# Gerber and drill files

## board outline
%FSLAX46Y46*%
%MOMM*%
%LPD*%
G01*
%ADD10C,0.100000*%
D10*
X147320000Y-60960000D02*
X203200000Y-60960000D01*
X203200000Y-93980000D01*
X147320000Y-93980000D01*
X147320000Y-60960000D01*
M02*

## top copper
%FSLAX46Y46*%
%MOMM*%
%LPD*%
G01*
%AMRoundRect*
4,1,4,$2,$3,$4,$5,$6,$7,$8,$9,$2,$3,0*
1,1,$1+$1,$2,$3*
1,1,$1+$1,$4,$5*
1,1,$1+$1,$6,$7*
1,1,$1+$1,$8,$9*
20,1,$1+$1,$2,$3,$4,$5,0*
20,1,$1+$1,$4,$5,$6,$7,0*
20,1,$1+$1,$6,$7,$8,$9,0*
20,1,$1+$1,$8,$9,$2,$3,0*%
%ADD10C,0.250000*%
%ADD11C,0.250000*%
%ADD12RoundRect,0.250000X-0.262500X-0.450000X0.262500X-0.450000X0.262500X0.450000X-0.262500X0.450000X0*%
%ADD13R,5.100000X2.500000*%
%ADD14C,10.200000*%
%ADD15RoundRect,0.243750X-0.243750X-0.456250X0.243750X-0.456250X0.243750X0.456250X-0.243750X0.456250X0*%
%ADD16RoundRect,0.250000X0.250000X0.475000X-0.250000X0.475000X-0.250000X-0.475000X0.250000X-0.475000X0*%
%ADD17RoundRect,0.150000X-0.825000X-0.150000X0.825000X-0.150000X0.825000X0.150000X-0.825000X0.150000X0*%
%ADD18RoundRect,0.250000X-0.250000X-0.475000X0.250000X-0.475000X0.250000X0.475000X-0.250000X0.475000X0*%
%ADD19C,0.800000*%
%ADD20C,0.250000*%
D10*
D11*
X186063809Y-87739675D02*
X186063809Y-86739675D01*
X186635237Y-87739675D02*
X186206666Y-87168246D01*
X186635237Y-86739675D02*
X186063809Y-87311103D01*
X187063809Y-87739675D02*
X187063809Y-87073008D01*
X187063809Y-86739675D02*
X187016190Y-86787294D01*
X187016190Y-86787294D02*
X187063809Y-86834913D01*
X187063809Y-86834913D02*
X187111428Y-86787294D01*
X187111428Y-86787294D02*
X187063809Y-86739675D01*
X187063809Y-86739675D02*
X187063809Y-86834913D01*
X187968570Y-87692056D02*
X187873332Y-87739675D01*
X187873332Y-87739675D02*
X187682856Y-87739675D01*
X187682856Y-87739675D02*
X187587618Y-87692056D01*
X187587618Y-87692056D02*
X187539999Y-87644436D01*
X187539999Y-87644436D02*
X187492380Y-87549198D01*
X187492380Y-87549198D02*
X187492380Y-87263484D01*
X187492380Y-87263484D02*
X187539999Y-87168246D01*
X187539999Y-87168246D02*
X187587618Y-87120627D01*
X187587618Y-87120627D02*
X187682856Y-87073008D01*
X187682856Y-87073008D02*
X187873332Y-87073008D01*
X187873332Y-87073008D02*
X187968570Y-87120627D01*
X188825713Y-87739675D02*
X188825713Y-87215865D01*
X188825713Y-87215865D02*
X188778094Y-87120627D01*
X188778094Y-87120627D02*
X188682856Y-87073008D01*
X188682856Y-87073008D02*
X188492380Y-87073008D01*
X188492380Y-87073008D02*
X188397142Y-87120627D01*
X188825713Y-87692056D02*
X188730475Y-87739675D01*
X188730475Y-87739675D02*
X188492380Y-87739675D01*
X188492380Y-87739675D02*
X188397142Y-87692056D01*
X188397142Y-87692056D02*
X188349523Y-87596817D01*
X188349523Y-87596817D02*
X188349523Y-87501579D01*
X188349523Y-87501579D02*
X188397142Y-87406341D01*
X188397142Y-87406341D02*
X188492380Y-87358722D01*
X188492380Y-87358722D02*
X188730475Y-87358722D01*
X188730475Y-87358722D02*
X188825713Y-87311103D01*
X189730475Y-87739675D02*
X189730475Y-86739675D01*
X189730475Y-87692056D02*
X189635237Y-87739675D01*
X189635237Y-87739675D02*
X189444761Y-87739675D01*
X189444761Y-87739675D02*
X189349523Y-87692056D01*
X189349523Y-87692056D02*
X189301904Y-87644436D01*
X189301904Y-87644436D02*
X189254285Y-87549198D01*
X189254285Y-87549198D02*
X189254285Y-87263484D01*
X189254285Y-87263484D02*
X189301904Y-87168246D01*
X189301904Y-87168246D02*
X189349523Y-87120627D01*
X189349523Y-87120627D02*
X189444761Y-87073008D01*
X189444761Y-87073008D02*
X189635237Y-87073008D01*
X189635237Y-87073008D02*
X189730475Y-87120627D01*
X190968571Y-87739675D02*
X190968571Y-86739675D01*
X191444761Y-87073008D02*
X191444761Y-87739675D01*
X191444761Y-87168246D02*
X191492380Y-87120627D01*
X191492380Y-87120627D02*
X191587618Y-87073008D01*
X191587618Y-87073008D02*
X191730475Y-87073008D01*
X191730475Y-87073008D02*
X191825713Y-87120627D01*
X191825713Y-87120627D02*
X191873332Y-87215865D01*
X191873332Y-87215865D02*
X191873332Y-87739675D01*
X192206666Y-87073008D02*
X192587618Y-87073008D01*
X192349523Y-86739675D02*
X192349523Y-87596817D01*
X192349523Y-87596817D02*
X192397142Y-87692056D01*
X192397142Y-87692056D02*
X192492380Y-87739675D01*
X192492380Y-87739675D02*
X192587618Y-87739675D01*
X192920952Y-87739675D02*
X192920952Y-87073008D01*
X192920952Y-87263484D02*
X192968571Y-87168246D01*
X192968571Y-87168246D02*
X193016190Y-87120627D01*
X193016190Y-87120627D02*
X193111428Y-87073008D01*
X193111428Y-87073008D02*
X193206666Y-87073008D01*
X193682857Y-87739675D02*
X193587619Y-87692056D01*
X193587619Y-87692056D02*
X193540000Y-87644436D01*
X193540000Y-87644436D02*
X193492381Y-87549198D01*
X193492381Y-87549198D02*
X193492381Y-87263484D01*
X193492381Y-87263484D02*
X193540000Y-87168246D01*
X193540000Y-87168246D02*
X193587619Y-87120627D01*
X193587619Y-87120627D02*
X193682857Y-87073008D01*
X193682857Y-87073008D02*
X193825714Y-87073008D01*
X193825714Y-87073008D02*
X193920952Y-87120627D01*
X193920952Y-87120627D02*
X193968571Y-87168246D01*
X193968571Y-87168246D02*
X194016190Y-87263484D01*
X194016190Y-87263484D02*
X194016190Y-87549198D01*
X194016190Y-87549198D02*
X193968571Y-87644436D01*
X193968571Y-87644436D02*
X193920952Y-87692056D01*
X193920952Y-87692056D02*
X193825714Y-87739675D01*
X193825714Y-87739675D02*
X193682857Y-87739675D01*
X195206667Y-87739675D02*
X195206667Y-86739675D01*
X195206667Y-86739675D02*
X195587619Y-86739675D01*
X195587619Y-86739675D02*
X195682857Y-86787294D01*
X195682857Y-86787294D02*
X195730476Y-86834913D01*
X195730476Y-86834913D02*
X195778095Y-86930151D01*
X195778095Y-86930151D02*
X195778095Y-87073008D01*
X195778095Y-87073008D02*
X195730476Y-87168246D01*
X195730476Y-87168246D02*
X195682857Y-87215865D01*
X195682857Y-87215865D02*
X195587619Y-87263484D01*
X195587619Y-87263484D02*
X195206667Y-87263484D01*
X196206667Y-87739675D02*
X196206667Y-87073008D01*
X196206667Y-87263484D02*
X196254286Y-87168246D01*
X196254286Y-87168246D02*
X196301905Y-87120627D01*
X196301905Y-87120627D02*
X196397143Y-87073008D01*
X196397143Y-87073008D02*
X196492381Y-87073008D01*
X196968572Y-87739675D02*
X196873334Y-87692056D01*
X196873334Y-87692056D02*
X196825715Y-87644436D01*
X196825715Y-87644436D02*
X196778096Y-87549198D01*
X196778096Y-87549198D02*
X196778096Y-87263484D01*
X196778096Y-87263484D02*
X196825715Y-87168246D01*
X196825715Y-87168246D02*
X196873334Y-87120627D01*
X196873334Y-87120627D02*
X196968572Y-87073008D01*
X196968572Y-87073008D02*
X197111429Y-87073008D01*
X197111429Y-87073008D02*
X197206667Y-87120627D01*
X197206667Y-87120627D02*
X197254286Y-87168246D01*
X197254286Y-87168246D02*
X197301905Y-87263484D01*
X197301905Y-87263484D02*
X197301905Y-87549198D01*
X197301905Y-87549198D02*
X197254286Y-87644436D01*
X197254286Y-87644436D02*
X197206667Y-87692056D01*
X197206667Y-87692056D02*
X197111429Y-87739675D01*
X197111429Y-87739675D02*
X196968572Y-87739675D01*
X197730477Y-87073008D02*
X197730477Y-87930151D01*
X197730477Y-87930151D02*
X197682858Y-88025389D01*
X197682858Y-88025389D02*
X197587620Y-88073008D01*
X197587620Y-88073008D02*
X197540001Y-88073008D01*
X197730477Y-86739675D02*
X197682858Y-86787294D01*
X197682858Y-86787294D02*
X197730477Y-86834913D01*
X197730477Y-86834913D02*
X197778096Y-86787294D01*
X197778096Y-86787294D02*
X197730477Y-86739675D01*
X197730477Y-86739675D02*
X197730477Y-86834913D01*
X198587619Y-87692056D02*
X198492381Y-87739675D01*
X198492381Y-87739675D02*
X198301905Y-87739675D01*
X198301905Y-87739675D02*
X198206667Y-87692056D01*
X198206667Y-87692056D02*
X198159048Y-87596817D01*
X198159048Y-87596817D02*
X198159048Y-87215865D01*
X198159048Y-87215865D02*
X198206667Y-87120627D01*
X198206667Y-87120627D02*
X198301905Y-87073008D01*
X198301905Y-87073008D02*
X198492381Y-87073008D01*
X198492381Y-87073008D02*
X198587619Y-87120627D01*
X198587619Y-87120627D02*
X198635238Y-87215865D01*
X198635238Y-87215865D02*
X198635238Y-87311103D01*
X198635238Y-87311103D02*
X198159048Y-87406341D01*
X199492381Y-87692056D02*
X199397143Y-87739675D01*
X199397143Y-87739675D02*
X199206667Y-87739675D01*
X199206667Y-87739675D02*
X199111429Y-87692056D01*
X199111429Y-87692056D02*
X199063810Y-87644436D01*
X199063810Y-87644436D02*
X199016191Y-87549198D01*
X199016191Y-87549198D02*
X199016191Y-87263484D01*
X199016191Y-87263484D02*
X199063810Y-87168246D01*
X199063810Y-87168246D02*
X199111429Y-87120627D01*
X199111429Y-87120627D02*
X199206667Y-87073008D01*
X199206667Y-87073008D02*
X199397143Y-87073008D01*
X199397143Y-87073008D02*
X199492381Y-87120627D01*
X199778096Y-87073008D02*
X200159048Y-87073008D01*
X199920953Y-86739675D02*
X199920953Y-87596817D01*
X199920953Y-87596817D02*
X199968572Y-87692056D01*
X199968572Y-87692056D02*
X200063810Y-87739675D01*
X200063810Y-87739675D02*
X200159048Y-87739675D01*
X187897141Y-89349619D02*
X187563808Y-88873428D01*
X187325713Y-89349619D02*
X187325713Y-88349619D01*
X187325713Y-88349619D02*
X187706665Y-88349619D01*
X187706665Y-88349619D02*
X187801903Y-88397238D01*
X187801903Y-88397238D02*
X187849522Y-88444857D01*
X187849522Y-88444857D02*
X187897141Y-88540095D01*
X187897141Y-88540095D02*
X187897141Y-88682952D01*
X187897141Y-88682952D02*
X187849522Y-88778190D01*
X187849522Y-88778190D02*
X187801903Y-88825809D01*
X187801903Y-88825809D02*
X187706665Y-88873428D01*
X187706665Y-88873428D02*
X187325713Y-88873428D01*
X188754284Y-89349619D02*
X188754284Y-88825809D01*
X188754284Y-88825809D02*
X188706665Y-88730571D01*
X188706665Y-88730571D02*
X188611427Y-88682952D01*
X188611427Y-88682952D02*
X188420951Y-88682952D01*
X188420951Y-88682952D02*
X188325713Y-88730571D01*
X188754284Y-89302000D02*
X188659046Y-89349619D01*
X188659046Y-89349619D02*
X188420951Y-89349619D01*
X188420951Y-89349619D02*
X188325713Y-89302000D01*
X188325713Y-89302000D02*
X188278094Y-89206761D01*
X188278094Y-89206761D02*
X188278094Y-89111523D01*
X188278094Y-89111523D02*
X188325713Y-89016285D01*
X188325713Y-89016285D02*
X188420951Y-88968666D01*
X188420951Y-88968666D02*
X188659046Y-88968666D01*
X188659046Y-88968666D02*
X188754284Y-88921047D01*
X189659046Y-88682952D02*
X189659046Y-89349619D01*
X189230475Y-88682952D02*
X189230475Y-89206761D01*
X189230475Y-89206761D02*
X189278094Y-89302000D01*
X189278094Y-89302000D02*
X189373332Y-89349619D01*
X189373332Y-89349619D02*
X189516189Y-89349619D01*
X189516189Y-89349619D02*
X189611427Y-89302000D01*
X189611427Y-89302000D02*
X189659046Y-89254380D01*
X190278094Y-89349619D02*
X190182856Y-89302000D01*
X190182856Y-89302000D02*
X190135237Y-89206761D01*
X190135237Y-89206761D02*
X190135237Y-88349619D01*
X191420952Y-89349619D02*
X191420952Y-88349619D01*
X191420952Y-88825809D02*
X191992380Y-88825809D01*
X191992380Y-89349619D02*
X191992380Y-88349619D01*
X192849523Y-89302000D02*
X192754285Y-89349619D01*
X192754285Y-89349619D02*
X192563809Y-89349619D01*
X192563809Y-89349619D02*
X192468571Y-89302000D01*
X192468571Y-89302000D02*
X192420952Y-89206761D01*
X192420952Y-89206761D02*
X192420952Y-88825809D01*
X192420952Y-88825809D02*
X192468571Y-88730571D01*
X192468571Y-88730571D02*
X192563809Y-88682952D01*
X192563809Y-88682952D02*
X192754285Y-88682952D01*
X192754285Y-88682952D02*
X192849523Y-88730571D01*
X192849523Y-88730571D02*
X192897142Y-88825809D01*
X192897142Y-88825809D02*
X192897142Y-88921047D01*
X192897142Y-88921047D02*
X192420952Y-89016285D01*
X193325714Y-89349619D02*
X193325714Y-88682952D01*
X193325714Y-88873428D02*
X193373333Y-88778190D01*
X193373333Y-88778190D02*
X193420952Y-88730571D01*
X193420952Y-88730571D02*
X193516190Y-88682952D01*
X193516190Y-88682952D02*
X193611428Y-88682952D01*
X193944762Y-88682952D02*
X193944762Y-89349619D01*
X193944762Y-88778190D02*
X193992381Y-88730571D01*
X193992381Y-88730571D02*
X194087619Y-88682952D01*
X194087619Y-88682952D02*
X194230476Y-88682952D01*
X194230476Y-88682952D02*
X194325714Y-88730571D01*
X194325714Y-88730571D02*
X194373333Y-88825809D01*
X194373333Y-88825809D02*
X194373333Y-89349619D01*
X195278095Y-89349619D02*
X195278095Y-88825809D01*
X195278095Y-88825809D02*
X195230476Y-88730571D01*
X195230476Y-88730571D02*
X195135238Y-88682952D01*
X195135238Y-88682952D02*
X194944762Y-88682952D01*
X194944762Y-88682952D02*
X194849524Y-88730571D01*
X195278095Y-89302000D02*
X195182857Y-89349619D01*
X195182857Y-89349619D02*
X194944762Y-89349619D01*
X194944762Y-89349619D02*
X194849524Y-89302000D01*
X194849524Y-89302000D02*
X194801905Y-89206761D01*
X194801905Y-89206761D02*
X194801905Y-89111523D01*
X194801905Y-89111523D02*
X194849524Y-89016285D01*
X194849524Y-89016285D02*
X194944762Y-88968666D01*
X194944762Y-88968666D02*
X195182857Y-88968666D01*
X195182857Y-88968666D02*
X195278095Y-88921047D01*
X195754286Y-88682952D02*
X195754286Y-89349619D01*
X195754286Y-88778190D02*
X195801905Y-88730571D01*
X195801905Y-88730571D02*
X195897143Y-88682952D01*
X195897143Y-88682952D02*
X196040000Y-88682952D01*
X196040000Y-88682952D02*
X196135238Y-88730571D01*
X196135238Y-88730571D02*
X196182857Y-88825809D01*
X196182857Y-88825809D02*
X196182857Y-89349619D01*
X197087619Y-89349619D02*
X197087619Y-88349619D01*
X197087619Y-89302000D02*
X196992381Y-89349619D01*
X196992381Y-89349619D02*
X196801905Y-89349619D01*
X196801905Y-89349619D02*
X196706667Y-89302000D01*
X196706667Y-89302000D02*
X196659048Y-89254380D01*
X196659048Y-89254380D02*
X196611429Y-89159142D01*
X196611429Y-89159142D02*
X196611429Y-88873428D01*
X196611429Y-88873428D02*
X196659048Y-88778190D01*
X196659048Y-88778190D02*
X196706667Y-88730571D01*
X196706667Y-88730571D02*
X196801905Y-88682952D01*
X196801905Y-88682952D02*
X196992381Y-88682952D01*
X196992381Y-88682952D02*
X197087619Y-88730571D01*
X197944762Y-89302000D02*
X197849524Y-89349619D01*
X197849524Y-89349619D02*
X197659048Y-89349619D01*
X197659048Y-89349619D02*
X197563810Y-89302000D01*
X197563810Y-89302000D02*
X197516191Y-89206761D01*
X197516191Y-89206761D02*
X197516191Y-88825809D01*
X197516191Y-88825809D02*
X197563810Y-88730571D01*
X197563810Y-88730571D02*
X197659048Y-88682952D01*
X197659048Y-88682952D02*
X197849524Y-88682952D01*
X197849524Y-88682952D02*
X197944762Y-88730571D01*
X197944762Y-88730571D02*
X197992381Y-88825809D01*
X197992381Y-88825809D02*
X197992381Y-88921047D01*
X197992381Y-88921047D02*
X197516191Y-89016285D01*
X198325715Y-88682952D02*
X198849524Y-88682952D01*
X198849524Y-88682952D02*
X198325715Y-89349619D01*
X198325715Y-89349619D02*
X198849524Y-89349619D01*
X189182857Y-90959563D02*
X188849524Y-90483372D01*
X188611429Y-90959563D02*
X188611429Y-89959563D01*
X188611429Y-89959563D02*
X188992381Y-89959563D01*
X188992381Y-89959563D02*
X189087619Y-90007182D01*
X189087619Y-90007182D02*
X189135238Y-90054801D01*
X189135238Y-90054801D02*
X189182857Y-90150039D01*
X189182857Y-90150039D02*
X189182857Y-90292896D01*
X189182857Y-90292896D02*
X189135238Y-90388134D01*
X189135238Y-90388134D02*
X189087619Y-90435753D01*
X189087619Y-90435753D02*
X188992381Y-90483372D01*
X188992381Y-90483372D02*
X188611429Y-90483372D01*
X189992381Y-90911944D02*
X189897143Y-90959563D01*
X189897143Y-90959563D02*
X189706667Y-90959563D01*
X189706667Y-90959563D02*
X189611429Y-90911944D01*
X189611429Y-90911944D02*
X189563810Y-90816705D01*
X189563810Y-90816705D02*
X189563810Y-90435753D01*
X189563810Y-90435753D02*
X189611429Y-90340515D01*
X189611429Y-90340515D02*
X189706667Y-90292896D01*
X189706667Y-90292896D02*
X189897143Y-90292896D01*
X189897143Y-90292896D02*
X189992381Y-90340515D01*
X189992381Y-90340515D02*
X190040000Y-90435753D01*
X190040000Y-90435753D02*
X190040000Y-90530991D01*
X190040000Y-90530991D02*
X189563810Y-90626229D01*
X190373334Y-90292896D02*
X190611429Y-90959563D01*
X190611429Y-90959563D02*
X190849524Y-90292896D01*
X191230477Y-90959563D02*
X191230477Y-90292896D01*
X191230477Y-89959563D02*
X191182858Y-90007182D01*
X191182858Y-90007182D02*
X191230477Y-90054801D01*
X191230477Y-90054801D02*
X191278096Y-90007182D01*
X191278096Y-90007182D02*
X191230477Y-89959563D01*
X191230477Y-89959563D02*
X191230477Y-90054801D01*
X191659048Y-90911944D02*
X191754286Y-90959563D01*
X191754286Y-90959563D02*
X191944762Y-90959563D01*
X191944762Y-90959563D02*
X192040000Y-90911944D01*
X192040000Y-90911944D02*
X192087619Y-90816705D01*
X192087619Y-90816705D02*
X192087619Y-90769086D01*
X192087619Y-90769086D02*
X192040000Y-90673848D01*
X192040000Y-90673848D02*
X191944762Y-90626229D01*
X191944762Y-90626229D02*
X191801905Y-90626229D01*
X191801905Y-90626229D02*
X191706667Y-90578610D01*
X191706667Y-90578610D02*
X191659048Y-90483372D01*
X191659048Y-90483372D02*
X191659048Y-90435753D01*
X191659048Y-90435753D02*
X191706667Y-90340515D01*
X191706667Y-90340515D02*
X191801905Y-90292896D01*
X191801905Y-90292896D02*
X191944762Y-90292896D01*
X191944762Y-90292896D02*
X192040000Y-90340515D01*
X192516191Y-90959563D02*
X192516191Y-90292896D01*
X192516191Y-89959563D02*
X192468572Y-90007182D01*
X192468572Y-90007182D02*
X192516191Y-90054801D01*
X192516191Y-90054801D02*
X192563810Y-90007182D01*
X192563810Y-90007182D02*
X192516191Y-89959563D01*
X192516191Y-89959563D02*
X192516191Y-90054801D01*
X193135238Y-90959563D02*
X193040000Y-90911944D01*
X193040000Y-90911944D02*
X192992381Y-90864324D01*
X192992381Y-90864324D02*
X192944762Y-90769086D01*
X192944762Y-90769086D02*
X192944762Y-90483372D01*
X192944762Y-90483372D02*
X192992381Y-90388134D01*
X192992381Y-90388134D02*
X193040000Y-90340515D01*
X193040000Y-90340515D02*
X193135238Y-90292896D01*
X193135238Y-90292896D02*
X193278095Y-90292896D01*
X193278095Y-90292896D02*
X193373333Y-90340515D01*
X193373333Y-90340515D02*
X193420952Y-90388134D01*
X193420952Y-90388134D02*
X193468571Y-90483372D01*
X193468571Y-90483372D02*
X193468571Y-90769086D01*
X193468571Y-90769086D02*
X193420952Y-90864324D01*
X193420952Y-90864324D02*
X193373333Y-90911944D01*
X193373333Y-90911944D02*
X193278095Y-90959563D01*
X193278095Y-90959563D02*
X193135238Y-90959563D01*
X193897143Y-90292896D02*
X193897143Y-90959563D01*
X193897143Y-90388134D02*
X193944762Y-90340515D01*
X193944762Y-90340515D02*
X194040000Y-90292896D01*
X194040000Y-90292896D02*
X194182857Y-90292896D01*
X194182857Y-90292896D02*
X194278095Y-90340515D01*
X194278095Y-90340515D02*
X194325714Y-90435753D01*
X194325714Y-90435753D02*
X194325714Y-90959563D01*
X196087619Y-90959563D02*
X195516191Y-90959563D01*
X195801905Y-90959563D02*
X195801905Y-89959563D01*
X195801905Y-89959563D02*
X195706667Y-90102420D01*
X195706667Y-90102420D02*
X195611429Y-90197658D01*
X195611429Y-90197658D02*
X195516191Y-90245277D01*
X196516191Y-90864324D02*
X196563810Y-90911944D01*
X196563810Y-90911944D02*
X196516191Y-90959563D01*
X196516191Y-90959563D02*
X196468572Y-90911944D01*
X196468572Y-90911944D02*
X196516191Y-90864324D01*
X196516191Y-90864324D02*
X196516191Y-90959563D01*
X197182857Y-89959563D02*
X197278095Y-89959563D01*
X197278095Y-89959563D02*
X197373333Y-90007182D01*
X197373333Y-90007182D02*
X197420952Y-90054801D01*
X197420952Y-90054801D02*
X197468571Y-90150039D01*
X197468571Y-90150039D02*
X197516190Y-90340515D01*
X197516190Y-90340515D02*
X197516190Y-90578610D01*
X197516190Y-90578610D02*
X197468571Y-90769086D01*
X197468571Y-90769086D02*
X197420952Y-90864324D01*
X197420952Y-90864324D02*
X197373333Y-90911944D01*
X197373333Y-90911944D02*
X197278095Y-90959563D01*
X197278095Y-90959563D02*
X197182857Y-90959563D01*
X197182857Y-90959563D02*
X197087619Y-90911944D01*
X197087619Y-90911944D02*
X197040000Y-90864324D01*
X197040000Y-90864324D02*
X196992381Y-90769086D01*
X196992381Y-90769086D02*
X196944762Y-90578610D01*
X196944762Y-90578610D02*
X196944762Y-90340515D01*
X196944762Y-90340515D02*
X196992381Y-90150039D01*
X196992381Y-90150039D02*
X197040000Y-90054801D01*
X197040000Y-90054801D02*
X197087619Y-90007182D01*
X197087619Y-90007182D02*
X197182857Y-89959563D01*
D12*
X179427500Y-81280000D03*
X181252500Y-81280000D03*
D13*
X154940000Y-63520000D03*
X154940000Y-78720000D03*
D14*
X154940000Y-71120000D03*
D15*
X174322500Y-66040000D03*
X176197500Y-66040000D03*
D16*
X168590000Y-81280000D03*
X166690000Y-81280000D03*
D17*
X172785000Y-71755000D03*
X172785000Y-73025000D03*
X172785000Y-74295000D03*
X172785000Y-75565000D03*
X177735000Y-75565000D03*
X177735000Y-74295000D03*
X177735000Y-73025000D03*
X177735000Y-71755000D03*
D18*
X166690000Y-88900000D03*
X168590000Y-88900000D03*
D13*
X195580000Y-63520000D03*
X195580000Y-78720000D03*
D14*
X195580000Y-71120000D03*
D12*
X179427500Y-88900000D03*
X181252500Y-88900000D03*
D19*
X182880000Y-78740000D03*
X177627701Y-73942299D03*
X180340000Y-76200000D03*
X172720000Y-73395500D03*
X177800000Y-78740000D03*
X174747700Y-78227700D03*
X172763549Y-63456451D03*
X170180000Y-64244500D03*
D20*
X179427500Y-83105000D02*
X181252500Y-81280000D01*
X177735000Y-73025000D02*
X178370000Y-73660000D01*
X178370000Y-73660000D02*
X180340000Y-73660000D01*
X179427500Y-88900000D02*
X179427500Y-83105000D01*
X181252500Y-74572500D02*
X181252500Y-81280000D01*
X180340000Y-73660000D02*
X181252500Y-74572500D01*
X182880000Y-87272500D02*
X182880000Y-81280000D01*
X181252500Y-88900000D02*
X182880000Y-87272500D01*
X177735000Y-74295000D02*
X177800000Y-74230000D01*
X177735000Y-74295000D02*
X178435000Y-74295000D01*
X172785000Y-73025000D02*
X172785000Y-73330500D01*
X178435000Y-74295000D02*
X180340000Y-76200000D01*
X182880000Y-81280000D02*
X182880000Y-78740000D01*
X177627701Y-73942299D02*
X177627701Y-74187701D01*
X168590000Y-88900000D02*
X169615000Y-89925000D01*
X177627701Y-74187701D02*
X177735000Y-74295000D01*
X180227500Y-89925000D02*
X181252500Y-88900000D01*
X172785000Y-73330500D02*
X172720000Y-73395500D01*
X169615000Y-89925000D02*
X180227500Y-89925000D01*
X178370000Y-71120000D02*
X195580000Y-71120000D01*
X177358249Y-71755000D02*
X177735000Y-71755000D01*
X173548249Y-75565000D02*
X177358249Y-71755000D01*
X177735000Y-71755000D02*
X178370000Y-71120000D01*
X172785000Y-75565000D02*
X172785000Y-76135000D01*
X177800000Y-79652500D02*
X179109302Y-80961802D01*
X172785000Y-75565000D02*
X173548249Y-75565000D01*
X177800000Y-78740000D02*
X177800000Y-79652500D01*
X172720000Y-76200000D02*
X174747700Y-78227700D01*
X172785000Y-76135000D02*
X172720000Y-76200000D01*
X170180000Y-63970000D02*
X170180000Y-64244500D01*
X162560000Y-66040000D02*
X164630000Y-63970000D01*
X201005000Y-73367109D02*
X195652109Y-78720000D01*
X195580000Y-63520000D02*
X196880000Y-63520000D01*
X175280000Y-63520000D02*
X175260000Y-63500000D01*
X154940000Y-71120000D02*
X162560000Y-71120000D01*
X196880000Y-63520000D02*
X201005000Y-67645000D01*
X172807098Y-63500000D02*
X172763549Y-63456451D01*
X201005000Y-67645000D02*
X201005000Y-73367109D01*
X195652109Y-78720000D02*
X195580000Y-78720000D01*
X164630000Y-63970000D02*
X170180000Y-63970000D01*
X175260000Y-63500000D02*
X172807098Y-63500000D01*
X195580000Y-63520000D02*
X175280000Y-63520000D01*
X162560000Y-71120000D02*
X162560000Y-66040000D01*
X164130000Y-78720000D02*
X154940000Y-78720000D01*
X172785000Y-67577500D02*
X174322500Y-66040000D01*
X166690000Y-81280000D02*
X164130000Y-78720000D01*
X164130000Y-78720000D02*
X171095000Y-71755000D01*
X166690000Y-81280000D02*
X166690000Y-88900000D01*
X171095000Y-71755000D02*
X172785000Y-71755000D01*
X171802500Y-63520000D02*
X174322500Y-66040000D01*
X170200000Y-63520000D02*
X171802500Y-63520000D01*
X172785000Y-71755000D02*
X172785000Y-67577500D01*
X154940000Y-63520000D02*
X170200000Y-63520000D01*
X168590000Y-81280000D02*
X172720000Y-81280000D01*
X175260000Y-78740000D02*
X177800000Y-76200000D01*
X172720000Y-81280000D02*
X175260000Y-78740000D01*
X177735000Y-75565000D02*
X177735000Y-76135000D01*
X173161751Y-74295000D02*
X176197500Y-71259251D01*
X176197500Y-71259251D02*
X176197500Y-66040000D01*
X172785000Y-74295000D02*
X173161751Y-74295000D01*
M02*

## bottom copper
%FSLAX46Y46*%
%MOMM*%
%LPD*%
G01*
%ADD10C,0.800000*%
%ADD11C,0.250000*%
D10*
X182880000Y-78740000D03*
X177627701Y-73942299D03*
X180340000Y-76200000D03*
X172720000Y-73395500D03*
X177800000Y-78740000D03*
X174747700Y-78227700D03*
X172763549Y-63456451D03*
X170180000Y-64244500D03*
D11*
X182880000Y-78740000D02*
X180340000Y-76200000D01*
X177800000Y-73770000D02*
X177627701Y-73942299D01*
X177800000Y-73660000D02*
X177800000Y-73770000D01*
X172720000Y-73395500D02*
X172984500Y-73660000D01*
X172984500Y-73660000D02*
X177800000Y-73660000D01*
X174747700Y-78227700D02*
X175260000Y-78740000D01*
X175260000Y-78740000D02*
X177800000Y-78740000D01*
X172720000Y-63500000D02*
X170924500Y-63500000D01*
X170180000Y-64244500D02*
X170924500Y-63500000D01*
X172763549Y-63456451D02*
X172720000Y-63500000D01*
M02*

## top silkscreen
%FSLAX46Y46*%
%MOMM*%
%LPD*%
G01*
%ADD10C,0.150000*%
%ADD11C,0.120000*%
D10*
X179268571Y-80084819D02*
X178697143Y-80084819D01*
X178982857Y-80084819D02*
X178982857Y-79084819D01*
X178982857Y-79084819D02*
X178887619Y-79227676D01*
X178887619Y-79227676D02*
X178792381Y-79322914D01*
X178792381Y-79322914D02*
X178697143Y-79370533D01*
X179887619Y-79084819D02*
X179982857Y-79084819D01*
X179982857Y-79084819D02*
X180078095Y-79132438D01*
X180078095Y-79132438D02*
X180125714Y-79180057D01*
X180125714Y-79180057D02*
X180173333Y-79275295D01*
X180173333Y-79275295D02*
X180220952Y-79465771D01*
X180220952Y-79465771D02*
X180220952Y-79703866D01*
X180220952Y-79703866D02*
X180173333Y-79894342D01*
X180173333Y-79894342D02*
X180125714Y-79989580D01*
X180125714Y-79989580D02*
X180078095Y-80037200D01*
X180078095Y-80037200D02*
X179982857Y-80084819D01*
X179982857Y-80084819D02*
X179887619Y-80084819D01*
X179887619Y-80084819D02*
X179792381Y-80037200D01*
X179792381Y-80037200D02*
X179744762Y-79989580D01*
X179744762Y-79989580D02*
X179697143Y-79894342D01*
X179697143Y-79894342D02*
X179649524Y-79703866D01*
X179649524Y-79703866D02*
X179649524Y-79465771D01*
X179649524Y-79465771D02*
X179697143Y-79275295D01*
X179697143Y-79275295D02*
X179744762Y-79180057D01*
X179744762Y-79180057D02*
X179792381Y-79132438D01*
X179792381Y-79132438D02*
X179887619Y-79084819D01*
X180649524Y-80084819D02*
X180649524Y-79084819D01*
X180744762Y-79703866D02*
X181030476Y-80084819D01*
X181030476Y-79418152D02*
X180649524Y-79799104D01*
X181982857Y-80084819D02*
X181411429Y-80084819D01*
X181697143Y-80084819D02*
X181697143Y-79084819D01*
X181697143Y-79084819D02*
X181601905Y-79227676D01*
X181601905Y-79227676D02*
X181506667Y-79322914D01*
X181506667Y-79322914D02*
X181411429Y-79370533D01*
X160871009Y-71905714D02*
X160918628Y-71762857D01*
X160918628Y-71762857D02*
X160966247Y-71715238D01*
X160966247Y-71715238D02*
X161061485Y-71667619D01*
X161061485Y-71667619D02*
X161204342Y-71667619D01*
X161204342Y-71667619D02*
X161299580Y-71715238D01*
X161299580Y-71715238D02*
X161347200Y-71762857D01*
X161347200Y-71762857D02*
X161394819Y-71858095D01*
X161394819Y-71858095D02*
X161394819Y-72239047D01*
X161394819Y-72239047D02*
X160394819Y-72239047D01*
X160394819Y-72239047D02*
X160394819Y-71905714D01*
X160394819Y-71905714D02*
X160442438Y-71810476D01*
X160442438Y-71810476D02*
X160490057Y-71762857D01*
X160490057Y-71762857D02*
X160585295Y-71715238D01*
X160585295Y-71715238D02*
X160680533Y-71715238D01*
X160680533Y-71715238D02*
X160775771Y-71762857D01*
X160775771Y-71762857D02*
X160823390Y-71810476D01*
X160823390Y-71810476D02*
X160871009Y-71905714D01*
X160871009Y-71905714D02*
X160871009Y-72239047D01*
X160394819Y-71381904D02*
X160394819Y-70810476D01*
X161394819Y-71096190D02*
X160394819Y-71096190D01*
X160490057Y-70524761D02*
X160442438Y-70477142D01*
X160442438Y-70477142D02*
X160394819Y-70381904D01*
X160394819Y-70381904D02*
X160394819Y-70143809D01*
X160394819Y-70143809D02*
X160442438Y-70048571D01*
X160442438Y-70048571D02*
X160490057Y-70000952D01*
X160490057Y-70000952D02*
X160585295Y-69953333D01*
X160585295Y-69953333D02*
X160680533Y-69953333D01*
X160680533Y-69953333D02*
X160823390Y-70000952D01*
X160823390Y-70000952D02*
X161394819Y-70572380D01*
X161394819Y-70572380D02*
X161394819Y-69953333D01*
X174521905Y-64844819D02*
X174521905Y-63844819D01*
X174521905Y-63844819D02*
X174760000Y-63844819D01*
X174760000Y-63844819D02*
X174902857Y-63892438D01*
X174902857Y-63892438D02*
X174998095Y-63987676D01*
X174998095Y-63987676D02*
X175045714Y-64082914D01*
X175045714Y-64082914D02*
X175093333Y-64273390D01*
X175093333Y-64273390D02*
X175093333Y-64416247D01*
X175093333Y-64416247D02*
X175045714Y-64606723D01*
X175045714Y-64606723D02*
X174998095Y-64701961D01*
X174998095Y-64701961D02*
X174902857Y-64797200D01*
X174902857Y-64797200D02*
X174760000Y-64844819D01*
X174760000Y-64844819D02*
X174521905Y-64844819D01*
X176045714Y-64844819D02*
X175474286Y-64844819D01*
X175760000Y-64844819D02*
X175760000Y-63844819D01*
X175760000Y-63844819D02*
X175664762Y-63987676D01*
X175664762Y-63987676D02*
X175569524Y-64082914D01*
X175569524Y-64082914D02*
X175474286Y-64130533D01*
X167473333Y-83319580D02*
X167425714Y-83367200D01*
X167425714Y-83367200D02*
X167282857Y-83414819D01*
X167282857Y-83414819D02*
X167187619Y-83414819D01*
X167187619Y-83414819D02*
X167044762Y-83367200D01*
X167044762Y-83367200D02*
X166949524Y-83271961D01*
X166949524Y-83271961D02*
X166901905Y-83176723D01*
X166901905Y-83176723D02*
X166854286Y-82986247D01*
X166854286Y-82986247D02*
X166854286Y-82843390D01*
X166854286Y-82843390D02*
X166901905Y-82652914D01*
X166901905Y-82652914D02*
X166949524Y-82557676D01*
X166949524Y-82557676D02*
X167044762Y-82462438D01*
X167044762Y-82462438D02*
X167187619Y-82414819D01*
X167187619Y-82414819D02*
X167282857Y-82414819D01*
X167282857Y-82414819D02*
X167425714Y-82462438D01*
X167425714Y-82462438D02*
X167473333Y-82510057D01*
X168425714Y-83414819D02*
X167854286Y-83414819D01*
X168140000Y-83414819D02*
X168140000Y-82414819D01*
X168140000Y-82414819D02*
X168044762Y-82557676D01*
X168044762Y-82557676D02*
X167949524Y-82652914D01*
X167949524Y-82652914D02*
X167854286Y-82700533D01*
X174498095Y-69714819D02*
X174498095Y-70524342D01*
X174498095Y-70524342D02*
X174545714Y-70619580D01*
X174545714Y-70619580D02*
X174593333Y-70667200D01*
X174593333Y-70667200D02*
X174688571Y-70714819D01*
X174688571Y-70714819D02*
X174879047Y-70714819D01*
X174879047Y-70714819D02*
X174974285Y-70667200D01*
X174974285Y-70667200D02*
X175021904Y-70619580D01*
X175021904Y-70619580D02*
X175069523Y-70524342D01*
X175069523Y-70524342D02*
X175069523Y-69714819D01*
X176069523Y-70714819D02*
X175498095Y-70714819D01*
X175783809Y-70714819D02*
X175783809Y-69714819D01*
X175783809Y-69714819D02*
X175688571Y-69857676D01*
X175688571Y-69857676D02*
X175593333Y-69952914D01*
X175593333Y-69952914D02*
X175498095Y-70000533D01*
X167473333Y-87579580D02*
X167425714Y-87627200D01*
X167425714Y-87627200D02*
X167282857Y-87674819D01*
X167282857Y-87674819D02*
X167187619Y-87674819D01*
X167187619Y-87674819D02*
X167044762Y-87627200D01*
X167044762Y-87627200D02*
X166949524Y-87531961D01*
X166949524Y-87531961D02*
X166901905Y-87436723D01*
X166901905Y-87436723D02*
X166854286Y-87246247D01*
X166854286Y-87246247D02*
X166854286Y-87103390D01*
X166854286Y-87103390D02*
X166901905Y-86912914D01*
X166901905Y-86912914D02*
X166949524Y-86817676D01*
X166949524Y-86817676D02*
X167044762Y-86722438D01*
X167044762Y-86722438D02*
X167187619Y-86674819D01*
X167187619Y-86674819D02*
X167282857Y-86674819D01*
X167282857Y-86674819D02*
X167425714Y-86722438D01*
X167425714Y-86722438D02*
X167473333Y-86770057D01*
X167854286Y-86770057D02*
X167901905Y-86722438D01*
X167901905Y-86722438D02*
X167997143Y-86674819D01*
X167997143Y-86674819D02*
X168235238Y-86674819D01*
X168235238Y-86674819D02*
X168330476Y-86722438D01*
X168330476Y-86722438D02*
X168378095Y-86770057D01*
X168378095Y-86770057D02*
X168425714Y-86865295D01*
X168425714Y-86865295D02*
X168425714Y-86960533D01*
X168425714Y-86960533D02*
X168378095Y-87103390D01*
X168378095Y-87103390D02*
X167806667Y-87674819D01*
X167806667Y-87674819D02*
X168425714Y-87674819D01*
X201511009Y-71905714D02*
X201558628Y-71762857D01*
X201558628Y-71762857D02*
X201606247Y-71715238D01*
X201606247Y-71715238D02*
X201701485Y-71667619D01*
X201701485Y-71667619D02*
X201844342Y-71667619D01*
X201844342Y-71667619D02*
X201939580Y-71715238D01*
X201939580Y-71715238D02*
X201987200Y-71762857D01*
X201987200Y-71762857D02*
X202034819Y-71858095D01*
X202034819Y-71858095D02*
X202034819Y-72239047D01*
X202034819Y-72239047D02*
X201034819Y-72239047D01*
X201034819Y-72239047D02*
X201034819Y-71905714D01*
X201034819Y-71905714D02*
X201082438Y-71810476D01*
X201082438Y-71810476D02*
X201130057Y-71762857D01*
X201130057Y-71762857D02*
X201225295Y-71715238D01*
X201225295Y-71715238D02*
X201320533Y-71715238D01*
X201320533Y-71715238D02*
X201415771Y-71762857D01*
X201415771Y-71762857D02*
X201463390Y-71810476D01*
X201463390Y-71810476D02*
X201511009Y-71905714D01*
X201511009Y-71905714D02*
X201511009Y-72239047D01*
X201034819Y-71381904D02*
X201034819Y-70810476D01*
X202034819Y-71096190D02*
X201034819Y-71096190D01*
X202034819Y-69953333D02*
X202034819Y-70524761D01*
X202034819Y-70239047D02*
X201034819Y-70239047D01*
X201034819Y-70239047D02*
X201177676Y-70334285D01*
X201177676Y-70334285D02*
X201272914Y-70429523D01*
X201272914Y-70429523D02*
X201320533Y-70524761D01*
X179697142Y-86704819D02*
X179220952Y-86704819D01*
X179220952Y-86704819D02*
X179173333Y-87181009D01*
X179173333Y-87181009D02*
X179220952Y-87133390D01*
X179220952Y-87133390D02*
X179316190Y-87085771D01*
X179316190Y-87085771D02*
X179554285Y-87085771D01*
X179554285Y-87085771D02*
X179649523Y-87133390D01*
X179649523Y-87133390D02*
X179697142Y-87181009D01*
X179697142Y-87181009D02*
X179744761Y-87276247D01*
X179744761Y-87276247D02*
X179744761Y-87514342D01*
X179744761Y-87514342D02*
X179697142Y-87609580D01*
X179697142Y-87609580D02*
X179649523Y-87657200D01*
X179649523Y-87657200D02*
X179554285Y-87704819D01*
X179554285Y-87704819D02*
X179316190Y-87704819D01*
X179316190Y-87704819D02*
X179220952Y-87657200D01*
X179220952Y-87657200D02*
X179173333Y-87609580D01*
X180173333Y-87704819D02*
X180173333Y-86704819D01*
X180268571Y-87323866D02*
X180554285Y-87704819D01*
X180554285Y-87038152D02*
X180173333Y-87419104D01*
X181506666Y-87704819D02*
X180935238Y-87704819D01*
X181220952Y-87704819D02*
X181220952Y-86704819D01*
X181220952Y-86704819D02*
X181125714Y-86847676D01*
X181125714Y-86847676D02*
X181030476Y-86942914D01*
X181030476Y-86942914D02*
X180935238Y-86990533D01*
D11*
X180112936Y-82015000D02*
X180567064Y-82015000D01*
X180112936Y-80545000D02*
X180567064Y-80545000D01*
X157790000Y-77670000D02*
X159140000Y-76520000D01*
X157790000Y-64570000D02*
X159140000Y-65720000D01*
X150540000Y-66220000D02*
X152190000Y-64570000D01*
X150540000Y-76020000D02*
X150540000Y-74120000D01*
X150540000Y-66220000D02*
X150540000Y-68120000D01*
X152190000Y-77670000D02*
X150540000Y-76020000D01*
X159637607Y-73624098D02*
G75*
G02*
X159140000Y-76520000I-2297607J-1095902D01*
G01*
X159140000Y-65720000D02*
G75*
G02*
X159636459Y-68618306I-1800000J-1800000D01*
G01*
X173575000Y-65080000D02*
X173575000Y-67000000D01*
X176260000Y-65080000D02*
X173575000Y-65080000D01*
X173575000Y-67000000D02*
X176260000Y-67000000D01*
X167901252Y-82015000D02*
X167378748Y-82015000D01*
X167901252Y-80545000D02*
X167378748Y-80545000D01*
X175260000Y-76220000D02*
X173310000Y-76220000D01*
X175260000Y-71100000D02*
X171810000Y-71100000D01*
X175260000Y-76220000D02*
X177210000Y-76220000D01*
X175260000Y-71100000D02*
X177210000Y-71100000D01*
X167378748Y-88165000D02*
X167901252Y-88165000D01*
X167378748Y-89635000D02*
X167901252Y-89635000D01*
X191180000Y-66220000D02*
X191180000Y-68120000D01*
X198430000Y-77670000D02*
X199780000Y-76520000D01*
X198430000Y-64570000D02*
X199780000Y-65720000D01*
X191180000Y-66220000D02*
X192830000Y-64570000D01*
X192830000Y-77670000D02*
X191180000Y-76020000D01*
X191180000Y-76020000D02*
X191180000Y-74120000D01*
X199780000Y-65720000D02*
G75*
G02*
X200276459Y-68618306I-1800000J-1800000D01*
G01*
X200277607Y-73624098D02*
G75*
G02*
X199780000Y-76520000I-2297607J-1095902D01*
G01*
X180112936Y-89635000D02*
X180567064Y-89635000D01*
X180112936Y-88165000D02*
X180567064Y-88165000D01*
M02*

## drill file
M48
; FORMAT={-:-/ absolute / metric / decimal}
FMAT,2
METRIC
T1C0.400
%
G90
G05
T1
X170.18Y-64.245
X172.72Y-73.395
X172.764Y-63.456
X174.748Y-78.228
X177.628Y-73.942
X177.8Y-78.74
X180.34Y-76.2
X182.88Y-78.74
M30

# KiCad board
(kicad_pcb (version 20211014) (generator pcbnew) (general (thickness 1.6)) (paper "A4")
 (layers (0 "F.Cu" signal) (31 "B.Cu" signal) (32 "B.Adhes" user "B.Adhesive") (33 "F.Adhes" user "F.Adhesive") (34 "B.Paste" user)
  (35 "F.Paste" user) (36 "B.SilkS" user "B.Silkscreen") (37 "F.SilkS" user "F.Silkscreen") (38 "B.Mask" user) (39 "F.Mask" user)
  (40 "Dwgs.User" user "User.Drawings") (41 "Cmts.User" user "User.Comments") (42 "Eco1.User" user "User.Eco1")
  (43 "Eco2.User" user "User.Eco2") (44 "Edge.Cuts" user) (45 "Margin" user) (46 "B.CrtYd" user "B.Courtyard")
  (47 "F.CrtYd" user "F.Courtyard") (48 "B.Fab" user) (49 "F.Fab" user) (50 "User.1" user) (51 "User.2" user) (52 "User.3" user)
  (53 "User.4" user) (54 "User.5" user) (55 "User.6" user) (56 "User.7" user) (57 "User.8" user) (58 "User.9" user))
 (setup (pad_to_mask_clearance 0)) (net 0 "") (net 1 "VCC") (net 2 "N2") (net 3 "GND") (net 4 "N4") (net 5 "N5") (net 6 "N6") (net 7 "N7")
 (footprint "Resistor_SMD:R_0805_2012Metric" (layer "F.Cu") (at 180.34 81.28)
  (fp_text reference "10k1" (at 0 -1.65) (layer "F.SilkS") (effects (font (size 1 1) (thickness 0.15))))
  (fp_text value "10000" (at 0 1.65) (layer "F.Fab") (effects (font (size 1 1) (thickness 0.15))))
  (fp_line (start -0.227064 0.735) (end 0.227064 0.735) (layer "F.SilkS") (width 0.12))
  (fp_line (start -0.227064 -0.735) (end 0.227064 -0.735) (layer "F.SilkS") (width 0.12))
  (pad "1" smd roundrect (at -0.9125 0) (size 1.025 1.4) (layers "F.Cu" "F.Paste" "F.Mask") (roundrect_rratio 0.243902439) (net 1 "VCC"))
  (pad "2" smd roundrect (at 0.9125 0) (size 1.025 1.4) (layers "F.Cu" "F.Paste" "F.Mask") (roundrect_rratio 0.243902439) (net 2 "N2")))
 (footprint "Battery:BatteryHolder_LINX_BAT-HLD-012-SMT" (layer "F.Cu") (at 154.94 71.12 90)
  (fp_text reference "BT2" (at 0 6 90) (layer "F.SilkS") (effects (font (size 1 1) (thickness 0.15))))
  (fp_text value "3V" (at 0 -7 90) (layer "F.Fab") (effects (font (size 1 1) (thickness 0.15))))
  (fp_line (start -6.55 2.85) (end -5.4 4.2) (layer "F.SilkS") (width 0.12))
  (fp_line (start 6.55 2.85) (end 5.4 4.2) (layer "F.SilkS") (width 0.12))
  (fp_line (start 4.9 -4.4) (end 6.55 -2.75) (layer "F.SilkS") (width 0.12))
  (fp_line (start -4.9 -4.4) (end -3 -4.4) (layer "F.SilkS") (width 0.12))
  (fp_line (start 4.9 -4.4) (end 3 -4.4) (layer "F.SilkS") (width 0.12))
  (fp_line (start -6.55 -2.75) (end -4.9 -4.4) (layer "F.SilkS") (width 0.12))
  (fp_arc (start -2.504098 4.697607) (mid -4.031094 4.908816) (end -5.4 4.2) (layer "F.SilkS") (width 0.12))
  (fp_arc (start 5.4 4.2) (mid 4.029781 4.909041) (end 2.501694 4.696459) (layer "F.SilkS") (width 0.12))
  (pad "1" smd rect (at 7.6 0 90) (size 2.5 5.1) (layers "F.Cu" "F.Paste" "F.Mask") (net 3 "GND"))
  (pad "1" smd rect (at -7.6 0 90) (size 2.5 5.1) (layers "F.Cu" "F.Paste" "F.Mask") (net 3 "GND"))
  (pad "2" smd circle (at 0 0 90) (size 10.2 10.2) (layers "F.Cu" "F.Mask") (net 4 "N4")))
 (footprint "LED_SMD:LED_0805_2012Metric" (layer "F.Cu") (at 175.26 66.04)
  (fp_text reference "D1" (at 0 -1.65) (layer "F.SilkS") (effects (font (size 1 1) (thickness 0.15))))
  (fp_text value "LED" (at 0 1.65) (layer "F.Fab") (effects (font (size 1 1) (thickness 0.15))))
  (fp_line (start -1.685 -0.96) (end -1.685 0.96) (layer "F.SilkS") (width 0.12))
  (fp_line (start 1 -0.96) (end -1.685 -0.96) (layer "F.SilkS") (width 0.12))
  (fp_line (start -1.685 0.96) (end 1 0.96) (layer "F.SilkS") (width 0.12))
  (pad "1" smd roundrect (at -0.9375 0) (size 0.975 1.4) (layers "F.Cu" "F.Paste" "F.Mask") (roundrect_rratio 0.25) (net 3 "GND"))
  (pad "2" smd roundrect (at 0.9375 0) (size 0.975 1.4) (layers "F.Cu" "F.Paste" "F.Mask") (roundrect_rratio 0.25) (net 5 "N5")))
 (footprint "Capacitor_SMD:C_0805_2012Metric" (layer "F.Cu") (at 167.64 81.28 180)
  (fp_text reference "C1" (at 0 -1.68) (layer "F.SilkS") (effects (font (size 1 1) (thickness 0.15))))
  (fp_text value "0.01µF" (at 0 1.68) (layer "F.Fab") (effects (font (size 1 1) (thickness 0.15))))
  (fp_line (start -0.261252 -0.735) (end 0.261252 -0.735) (layer "F.SilkS") (width 0.12))
  (fp_line (start -0.261252 0.735) (end 0.261252 0.735) (layer "F.SilkS") (width 0.12))
  (pad "1" smd roundrect (at -0.95 0 180) (size 1 1.45) (layers "F.Cu" "F.Paste" "F.Mask") (roundrect_rratio 0.25) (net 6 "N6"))
  (pad "2" smd roundrect (at 0.95 0 180) (size 1 1.45) (layers "F.Cu" "F.Paste" "F.Mask") (roundrect_rratio 0.25) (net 3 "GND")))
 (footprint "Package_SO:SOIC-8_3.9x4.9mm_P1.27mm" (layer "F.Cu") (at 175.26 73.66)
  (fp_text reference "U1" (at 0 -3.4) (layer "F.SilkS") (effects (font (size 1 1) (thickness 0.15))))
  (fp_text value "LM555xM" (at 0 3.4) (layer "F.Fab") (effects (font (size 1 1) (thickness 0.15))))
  (fp_line (start 0 2.56) (end -1.95 2.56) (layer "F.SilkS") (width 0.12))
  (fp_line (start 0 -2.56) (end -3.45 -2.56) (layer "F.SilkS") (width 0.12))
  (fp_line (start 0 2.56) (end 1.95 2.56) (layer "F.SilkS") (width 0.12))
  (fp_line (start 0 -2.56) (end 1.95 -2.56) (layer "F.SilkS") (width 0.12))
  (pad "1" smd roundrect (at -2.475 -1.905) (size 1.95 0.6) (layers "F.Cu" "F.Paste" "F.Mask") (roundrect_rratio 0.25) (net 3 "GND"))
  (pad "2" smd roundrect (at -2.475 -0.635) (size 1.95 0.6) (layers "F.Cu" "F.Paste" "F.Mask") (roundrect_rratio 0.25) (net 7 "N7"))
  (pad "3" smd roundrect (at -2.475 0.635) (size 1.95 0.6) (layers "F.Cu" "F.Paste" "F.Mask") (roundrect_rratio 0.25) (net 5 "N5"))
  (pad "4" smd roundrect (at -2.475 1.905) (size 1.95 0.6) (layers "F.Cu" "F.Paste" "F.Mask") (roundrect_rratio 0.25) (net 1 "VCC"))
  (pad "5" smd roundrect (at 2.475 1.905) (size 1.95 0.6) (layers "F.Cu" "F.Paste" "F.Mask") (roundrect_rratio 0.25) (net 6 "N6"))
  (pad "6" smd roundrect (at 2.475 0.635) (size 1.95 0.6) (layers "F.Cu" "F.Paste" "F.Mask") (roundrect_rratio 0.25) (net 7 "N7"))
  (pad "7" smd roundrect (at 2.475 -0.635) (size 1.95 0.6) (layers "F.Cu" "F.Paste" "F.Mask") (roundrect_rratio 0.25) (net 2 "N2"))
  (pad "8" smd roundrect (at 2.475 -1.905) (size 1.95 0.6) (layers "F.Cu" "F.Paste" "F.Mask") (roundrect_rratio 0.25) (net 1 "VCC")))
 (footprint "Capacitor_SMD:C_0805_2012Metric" (layer "F.Cu") (at 167.64 88.9)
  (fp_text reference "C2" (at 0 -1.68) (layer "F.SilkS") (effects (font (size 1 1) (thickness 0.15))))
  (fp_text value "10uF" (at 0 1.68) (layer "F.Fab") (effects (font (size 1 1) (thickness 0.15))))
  (fp_line (start -0.261252 -0.735) (end 0.261252 -0.735) (layer "F.SilkS") (width 0.12))
  (fp_line (start -0.261252 0.735) (end 0.261252 0.735) (layer "F.SilkS") (width 0.12))
  (pad "1" smd roundrect (at -0.95 0) (size 1 1.45) (layers "F.Cu" "F.Paste" "F.Mask") (roundrect_rratio 0.25) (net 3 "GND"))
  (pad "2" smd roundrect (at 0.95 0) (size 1 1.45) (layers "F.Cu" "F.Paste" "F.Mask") (roundrect_rratio 0.25) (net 7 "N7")))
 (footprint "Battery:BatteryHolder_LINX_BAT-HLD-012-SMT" (layer "F.Cu") (at 195.58 71.12 90)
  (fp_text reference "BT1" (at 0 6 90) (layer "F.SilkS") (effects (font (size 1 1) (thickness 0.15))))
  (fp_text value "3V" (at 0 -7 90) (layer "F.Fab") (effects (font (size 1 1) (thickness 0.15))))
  (fp_line (start 4.9 -4.4) (end 3 -4.4) (layer "F.SilkS") (width 0.12))
  (fp_line (start -6.55 2.85) (end -5.4 4.2) (layer "F.SilkS") (width 0.12))
  (fp_line (start 6.55 2.85) (end 5.4 4.2) (layer "F.SilkS") (width 0.12))
  (fp_line (start 4.9 -4.4) (end 6.55 -2.75) (layer "F.SilkS") (width 0.12))
  (fp_line (start -6.55 -2.75) (end -4.9 -4.4) (layer "F.SilkS") (width 0.12))
  (fp_line (start -4.9 -4.4) (end -3 -4.4) (layer "F.SilkS") (width 0.12))
  (fp_arc (start 5.4 4.2) (mid 4.029781 4.909041) (end 2.501694 4.696459) (layer "F.SilkS") (width 0.12))
  (fp_arc (start -2.504098 4.697607) (mid -4.031094 4.908816) (end -5.4 4.2) (layer "F.SilkS") (width 0.12))
  (pad "1" smd rect (at 7.6 0 90) (size 2.5 5.1) (layers "F.Cu" "F.Paste" "F.Mask") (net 4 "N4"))
  (pad "1" smd rect (at -7.6 0 90) (size 2.5 5.1) (layers "F.Cu" "F.Paste" "F.Mask") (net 4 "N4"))
  (pad "2" smd circle (at 0 0 90) (size 10.2 10.2) (layers "F.Cu" "F.Mask") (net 1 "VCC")))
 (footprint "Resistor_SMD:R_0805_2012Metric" (layer "F.Cu") (at 180.34 88.9)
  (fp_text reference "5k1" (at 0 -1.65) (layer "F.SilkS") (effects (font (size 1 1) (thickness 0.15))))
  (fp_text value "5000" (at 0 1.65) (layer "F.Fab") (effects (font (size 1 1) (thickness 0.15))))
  (fp_line (start -0.227064 0.735) (end 0.227064 0.735) (layer "F.SilkS") (width 0.12))
  (fp_line (start -0.227064 -0.735) (end 0.227064 -0.735) (layer "F.SilkS") (width 0.12))
  (pad "1" smd roundrect (at -0.9125 0) (size 1.025 1.4) (layers "F.Cu" "F.Paste" "F.Mask") (roundrect_rratio 0.243902439) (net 2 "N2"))
  (pad "2" smd roundrect (at 0.9125 0) (size 1.025 1.4) (layers "F.Cu" "F.Paste" "F.Mask") (roundrect_rratio 0.243902439) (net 7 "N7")))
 (gr_rect (start 147.32 60.96) (end 203.2 93.98) (layer "Edge.Cuts") (width 0.1) (fill none))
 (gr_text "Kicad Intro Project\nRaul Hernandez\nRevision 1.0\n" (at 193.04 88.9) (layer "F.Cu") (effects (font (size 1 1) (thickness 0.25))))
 (segment (start 179.4275 83.105) (end 181.2525 81.28) (width 0.25) (layer "F.Cu") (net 2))
 (segment (start 177.735 73.025) (end 178.37 73.66) (width 0.25) (layer "F.Cu") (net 2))
 (segment (start 178.37 73.66) (end 180.34 73.66) (width 0.25) (layer "F.Cu") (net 2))
 (segment (start 179.4275 88.9) (end 179.4275 83.105) (width 0.25) (layer "F.Cu") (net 2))
 (segment (start 181.2525 74.5725) (end 181.2525 81.28) (width 0.25) (layer "F.Cu") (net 2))
 (segment (start 180.34 73.66) (end 181.2525 74.5725) (width 0.25) (layer "F.Cu") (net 2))
 (segment (start 182.88 87.2725) (end 182.88 81.28) (width 0.25) (layer "F.Cu") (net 7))
 (segment (start 181.2525 88.9) (end 182.88 87.2725) (width 0.25) (layer "F.Cu") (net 7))
 (segment (start 177.735 74.295) (end 177.8 74.23) (width 0.25) (layer "F.Cu") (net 7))
 (segment (start 177.735 74.295) (end 178.435 74.295) (width 0.25) (layer "F.Cu") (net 7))
 (segment (start 172.785 73.025) (end 172.785 73.3305) (width 0.25) (layer "F.Cu") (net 7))
 (segment (start 178.435 74.295) (end 180.34 76.2) (width 0.25) (layer "F.Cu") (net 7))
 (segment (start 182.88 81.28) (end 182.88 78.74) (width 0.25) (layer "F.Cu") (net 7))
 (segment (start 177.627701 73.942299) (end 177.627701 74.187701) (width 0.25) (layer "F.Cu") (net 7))
 (segment (start 168.59 88.9) (end 169.615 89.925) (width 0.25) (layer "F.Cu") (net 7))
 (segment (start 177.627701 74.187701) (end 177.735 74.295) (width 0.25) (layer "F.Cu") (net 7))
 (segment (start 180.2275 89.925) (end 181.2525 88.9) (width 0.25) (layer "F.Cu") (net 7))
 (segment (start 172.785 73.3305) (end 172.72 73.3955) (width 0.25) (layer "F.Cu") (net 7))
 (segment (start 169.615 89.925) (end 180.2275 89.925) (width 0.25) (layer "F.Cu") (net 7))
 (via (at 182.88 78.74) (size 0.8) (drill 0.4) (layers "F.Cu" "B.Cu") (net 7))
 (via (at 177.627701 73.942299) (size 0.8) (drill 0.4) (layers "F.Cu" "B.Cu") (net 7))
 (via (at 180.34 76.2) (size 0.8) (drill 0.4) (layers "F.Cu" "B.Cu") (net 7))
 (via (at 172.72 73.3955) (size 0.8) (drill 0.4) (layers "F.Cu" "B.Cu") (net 7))
 (segment (start 182.88 78.74) (end 180.34 76.2) (width 0.25) (layer "B.Cu") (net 7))
 (segment (start 177.8 73.77) (end 177.627701 73.942299) (width 0.25) (layer "B.Cu") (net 7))
 (segment (start 177.8 73.66) (end 177.8 73.77) (width 0.25) (layer "B.Cu") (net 7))
 (segment (start 172.72 73.3955) (end 172.9845 73.66) (width 0.25) (layer "B.Cu") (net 7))
 (segment (start 172.9845 73.66) (end 177.8 73.66) (width 0.25) (layer "B.Cu") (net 7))
 (segment (start 178.37 71.12) (end 195.58 71.12) (width 0.25) (layer "F.Cu") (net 1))
 (segment (start 177.358249 71.755) (end 177.735 71.755) (width 0.25) (layer "F.Cu") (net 1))
 (segment (start 173.548249 75.565) (end 177.358249 71.755) (width 0.25) (layer "F.Cu") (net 1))
 (segment (start 177.735 71.755) (end 178.37 71.12) (width 0.25) (layer "F.Cu") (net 1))
 (segment (start 172.785 75.565) (end 172.785 76.135) (width 0.25) (layer "F.Cu") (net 1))
 (segment (start 177.8 79.6525) (end 179.109302 80.961802) (width 0.25) (layer "F.Cu") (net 1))
 (segment (start 172.785 75.565) (end 173.548249 75.565) (width 0.25) (layer "F.Cu") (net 1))
 (segment (start 177.8 78.74) (end 177.8 79.6525) (width 0.25) (layer "F.Cu") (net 1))
 (segment (start 172.72 76.2) (end 174.7477 78.2277) (width 0.25) (layer "F.Cu") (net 1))
 (segment (start 172.785 76.135) (end 172.72 76.2) (width 0.25) (layer "F.Cu") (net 1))
 (via (at 177.8 78.74) (size 0.8) (drill 0.4) (layers "F.Cu" "B.Cu") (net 1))
 (via (at 174.7477 78.2277) (size 0.8) (drill 0.4) (layers "F.Cu" "B.Cu") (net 1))
 (segment (start 174.7477 78.2277) (end 175.26 78.74) (width 0.25) (layer "B.Cu") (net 1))
 (segment (start 175.26 78.74) (end 177.8 78.74) (width 0.25) (layer "B.Cu") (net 1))
 (segment (start 170.18 63.97) (end 170.18 64.2445) (width 0.25) (layer "F.Cu") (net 4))
 (segment (start 162.56 66.04) (end 164.63 63.97) (width 0.25) (layer "F.Cu") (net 4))
 (segment (start 201.005 73.367109) (end 195.652109 78.72) (width 0.25) (layer "F.Cu") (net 4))
 (segment (start 195.58 63.52) (end 196.88 63.52) (width 0.25) (layer "F.Cu") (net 4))
 (segment (start 175.28 63.52) (end 175.26 63.5) (width 0.25) (layer "F.Cu") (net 4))
 (segment (start 154.94 71.12) (end 162.56 71.12) (width 0.25) (layer "F.Cu") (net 4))
 (segment (start 196.88 63.52) (end 201.005 67.645) (width 0.25) (layer "F.Cu") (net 4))
 (segment (start 172.807098 63.5) (end 172.763549 63.456451) (width 0.25) (layer "F.Cu") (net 4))
 (segment (start 201.005 67.645) (end 201.005 73.367109) (width 0.25) (layer "F.Cu") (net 4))
 (segment (start 195.652109 78.72) (end 195.58 78.72) (width 0.25) (layer "F.Cu") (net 4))
 (segment (start 164.63 63.97) (end 170.18 63.97) (width 0.25) (layer "F.Cu") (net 4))
 (segment (start 175.26 63.5) (end 172.807098 63.5) (width 0.25) (layer "F.Cu") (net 4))
 (segment (start 195.58 63.52) (end 175.28 63.52) (width 0.25) (layer "F.Cu") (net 4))
 (segment (start 162.56 71.12) (end 162.56 66.04) (width 0.25) (layer "F.Cu") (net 4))
 (via (at 172.763549 63.456451) (size 0.8) (drill 0.4) (layers "F.Cu" "B.Cu") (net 4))
 (via (at 170.18 64.2445) (size 0.8) (drill 0.4) (layers "F.Cu" "B.Cu") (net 4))
 (segment (start 172.72 63.5) (end 170.9245 63.5) (width 0.25) (layer "B.Cu") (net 4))
 (segment (start 170.18 64.2445) (end 170.9245 63.5) (width 0.25) (layer "B.Cu") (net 4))
 (segment (start 172.763549 63.456451) (end 172.72 63.5) (width 0.25) (layer "B.Cu") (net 4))
 (segment (start 164.13 78.72) (end 154.94 78.72) (width 0.25) (layer "F.Cu") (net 3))
 (segment (start 172.785 67.5775) (end 174.3225 66.04) (width 0.25) (layer "F.Cu") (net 3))
 (segment (start 166.69 81.28) (end 164.13 78.72) (width 0.25) (layer "F.Cu") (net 3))
 (segment (start 164.13 78.72) (end 171.095 71.755) (width 0.25) (layer "F.Cu") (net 3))
 (segment (start 166.69 81.28) (end 166.69 88.9) (width 0.25) (layer "F.Cu") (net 3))
 (segment (start 171.095 71.755) (end 172.785 71.755) (width 0.25) (layer "F.Cu") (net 3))
 (segment (start 171.8025 63.52) (end 174.3225 66.04) (width 0.25) (layer "F.Cu") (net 3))
 (segment (start 170.2 63.52) (end 171.8025 63.52) (width 0.25) (layer "F.Cu") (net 3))
 (segment (start 172.785 71.755) (end 172.785 67.5775) (width 0.25) (layer "F.Cu") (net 3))
 (segment (start 154.94 63.52) (end 170.2 63.52) (width 0.25) (layer "F.Cu") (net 3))
 (segment (start 168.59 81.28) (end 172.72 81.28) (width 0.25) (layer "F.Cu") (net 6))
 (segment (start 175.26 78.74) (end 177.8 76.2) (width 0.25) (layer "F.Cu") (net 6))
 (segment (start 172.72 81.28) (end 175.26 78.74) (width 0.25) (layer "F.Cu") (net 6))
 (segment (start 177.735 75.565) (end 177.735 76.135) (width 0.25) (layer "F.Cu") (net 6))
 (segment (start 173.161751 74.295) (end 176.1975 71.259251) (width 0.25) (layer "F.Cu") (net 5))
 (segment (start 176.1975 71.259251) (end 176.1975 66.04) (width 0.25) (layer "F.Cu") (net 5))
 (segment (start 172.785 74.295) (end 173.161751 74.295) (width 0.25) (layer "F.Cu") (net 5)))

